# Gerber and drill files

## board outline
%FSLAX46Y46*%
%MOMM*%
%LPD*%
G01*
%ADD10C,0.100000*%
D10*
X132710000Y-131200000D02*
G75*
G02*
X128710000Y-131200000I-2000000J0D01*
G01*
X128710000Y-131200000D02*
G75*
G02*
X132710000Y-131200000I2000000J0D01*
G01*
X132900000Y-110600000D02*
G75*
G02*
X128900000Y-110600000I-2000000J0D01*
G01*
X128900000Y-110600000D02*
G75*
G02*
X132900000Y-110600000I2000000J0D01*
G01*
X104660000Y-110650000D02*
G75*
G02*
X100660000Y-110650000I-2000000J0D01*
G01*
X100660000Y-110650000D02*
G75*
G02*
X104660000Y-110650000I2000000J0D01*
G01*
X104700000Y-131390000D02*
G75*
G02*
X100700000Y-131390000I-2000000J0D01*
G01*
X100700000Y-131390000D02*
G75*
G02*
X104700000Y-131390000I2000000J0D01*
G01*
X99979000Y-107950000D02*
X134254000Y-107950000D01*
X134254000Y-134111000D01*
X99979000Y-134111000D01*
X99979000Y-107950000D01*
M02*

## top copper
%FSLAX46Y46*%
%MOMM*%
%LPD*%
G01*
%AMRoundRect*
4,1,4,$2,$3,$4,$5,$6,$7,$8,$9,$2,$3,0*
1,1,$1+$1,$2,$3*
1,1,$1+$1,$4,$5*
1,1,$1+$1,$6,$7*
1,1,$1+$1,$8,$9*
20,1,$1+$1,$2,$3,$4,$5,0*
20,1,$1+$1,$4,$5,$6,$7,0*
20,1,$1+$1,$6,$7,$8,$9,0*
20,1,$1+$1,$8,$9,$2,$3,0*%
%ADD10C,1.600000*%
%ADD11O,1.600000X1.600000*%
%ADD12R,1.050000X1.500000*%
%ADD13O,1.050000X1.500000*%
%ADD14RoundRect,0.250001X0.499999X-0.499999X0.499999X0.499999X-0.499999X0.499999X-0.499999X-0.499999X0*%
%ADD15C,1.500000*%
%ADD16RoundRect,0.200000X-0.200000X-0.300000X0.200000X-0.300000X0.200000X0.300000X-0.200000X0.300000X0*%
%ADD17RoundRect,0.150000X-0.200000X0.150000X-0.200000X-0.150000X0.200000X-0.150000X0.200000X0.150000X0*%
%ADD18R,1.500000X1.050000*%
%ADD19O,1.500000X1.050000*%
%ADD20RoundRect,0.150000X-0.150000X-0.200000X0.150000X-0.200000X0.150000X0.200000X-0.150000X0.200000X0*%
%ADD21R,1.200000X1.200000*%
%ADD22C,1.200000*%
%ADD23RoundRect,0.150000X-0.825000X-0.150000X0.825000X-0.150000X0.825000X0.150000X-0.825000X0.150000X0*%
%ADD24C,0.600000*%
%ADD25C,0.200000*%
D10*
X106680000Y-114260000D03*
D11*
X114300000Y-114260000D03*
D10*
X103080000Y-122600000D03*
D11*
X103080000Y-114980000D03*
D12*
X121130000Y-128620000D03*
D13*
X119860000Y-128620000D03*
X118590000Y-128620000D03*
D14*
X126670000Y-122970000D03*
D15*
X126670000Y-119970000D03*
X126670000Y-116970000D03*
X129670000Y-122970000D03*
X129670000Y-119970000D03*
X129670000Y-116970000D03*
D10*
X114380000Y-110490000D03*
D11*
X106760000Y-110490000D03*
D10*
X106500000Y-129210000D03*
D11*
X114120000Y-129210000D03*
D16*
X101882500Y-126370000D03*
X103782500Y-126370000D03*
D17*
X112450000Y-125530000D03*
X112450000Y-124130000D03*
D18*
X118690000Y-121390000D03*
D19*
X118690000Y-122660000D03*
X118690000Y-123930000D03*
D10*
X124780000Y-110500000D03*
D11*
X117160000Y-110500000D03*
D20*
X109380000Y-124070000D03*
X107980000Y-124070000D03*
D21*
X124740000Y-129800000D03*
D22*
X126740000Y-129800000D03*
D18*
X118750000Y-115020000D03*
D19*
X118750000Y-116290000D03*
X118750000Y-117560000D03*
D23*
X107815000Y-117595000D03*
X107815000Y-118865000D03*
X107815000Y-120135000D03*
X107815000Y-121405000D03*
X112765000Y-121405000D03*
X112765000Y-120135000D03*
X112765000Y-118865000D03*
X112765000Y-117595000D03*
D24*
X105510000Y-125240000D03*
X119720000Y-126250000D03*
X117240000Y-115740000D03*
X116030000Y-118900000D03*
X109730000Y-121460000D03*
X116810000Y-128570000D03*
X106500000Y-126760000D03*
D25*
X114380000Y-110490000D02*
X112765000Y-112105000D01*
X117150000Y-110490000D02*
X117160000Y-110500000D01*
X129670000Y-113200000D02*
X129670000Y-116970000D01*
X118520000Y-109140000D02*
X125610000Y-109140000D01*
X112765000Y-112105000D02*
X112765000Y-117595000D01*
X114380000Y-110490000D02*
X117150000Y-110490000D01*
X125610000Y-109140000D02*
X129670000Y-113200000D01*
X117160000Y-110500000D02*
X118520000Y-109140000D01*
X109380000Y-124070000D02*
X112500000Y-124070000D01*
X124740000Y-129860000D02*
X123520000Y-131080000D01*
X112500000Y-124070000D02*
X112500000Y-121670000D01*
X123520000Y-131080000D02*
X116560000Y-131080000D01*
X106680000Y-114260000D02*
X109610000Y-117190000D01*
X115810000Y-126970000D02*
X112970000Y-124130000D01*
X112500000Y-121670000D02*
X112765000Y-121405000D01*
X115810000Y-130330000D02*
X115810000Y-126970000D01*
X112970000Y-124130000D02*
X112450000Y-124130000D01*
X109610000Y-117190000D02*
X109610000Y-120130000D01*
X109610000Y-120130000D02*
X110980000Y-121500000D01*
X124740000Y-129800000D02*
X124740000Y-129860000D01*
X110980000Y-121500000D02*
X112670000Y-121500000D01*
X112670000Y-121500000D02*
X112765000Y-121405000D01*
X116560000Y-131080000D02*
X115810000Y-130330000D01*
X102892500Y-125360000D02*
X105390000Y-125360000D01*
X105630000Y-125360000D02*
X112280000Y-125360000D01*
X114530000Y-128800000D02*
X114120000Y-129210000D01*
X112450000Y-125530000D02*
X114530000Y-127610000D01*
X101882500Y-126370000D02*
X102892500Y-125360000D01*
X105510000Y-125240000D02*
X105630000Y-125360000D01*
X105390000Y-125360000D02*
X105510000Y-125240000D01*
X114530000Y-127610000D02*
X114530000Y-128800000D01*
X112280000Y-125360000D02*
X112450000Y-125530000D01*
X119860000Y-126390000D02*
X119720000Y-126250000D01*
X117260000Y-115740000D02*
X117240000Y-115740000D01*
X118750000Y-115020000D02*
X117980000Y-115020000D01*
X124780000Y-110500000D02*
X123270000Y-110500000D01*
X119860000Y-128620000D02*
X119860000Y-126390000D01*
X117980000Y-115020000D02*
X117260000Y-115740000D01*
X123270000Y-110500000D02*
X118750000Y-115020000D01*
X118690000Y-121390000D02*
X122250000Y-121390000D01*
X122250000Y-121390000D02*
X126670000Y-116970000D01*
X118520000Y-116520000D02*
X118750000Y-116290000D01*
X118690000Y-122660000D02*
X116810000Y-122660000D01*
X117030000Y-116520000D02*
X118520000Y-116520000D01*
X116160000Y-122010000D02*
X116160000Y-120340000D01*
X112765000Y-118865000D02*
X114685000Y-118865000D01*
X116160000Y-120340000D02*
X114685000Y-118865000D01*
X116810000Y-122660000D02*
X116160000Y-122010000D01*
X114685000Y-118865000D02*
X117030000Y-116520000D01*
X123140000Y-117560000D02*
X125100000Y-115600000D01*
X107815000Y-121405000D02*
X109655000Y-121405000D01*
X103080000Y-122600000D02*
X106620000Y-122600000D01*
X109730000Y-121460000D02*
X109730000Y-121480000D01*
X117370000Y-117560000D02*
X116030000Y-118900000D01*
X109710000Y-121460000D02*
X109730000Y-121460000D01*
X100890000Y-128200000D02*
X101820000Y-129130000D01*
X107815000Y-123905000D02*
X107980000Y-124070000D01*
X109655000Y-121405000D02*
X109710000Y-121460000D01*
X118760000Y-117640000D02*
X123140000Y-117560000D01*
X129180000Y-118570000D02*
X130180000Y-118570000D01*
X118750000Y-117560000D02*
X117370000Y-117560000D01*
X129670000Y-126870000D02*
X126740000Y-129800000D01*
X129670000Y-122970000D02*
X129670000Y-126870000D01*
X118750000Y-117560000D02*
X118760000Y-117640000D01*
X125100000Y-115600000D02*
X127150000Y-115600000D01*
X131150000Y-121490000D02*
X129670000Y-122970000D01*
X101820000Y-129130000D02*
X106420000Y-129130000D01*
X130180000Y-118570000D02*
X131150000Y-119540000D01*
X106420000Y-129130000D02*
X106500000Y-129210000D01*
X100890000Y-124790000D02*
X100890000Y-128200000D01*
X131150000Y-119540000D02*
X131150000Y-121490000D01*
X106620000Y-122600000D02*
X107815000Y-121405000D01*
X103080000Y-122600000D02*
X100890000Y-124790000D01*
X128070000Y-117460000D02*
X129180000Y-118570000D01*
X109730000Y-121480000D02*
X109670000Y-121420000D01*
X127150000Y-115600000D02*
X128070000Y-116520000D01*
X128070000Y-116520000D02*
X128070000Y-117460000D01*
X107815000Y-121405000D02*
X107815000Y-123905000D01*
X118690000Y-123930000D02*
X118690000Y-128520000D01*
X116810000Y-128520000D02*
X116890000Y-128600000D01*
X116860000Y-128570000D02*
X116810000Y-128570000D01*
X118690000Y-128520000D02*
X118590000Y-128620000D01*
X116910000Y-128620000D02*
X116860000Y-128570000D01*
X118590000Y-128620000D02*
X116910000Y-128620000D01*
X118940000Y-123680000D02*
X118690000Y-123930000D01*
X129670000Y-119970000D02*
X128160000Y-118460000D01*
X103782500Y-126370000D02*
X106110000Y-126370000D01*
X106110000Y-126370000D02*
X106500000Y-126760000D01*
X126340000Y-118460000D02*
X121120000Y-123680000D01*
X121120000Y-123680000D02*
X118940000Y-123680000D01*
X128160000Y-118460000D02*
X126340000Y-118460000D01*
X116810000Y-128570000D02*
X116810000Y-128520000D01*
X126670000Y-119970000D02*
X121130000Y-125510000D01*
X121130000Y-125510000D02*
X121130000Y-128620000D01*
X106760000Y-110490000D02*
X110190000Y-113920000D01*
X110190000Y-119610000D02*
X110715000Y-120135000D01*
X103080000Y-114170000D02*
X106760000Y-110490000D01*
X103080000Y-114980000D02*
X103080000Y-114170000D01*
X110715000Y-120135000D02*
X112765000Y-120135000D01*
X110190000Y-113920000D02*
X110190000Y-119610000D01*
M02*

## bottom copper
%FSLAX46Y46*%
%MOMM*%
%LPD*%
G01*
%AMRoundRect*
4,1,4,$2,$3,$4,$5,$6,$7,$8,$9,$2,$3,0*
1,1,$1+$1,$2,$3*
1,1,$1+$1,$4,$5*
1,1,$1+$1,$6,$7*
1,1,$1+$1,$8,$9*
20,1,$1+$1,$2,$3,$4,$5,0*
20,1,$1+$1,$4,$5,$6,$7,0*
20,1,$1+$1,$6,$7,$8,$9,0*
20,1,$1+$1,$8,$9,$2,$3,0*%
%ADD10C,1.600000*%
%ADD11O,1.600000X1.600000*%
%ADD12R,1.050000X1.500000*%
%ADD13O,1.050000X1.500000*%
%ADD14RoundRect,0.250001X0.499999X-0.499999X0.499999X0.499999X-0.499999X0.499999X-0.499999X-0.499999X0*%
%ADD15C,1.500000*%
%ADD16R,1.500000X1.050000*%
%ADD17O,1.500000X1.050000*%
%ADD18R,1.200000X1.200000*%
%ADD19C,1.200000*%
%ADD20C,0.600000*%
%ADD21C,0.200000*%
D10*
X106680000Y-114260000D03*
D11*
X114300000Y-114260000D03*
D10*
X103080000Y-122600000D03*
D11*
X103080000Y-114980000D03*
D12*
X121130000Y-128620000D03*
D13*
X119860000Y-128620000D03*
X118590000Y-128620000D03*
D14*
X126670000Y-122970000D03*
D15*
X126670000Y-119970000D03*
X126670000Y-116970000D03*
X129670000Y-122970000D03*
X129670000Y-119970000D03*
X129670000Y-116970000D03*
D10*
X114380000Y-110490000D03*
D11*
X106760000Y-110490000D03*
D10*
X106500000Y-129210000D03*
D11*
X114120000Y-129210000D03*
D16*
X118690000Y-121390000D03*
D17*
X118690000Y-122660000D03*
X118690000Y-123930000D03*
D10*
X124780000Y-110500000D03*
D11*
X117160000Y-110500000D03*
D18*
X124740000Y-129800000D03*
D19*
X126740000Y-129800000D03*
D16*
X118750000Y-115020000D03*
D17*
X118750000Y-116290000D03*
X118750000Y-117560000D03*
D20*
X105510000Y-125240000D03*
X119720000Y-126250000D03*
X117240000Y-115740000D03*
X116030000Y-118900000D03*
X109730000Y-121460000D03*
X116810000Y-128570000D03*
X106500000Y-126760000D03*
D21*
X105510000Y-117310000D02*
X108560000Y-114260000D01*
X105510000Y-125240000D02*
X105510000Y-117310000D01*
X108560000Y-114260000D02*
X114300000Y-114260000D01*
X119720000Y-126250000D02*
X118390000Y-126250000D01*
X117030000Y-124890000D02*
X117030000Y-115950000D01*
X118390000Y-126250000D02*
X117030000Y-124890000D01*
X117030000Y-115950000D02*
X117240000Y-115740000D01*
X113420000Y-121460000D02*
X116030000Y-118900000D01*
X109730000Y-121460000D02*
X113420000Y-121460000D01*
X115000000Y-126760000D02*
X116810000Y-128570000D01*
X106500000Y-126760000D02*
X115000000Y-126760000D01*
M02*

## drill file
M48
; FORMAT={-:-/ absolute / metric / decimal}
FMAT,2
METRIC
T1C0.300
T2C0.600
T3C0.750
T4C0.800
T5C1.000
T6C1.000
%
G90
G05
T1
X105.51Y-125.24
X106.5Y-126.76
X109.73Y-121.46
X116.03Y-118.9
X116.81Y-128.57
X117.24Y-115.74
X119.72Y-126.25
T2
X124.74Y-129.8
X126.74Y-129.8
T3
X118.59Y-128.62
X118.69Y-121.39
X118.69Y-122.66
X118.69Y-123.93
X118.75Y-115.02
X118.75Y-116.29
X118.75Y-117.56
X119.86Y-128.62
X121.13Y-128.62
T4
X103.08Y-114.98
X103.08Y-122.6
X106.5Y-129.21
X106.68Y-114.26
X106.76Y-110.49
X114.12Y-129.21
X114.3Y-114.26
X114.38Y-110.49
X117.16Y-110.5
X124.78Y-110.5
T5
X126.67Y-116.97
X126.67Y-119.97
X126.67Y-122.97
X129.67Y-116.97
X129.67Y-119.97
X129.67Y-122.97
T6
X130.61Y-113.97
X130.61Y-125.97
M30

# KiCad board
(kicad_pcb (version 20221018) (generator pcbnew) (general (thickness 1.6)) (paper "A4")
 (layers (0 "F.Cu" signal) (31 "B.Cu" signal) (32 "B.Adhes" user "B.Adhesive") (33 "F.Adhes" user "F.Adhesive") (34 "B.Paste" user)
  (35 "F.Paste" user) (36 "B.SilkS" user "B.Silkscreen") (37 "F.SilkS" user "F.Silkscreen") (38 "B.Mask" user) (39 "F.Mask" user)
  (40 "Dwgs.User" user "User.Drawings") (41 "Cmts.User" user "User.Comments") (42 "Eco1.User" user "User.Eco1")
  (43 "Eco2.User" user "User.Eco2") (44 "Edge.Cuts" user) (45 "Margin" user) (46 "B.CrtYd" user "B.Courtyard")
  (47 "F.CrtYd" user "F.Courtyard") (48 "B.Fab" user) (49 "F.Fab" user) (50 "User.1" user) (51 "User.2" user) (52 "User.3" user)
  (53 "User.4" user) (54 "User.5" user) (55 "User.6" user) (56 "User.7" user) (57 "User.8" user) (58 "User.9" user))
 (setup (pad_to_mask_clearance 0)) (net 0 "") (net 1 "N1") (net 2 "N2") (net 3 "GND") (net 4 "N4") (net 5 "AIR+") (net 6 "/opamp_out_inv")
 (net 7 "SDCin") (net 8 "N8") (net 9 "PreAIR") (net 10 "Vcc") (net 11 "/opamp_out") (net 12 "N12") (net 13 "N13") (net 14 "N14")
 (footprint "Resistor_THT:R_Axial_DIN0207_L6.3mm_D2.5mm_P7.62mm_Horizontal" (layer "F.Cu") (at 106.68 114.26)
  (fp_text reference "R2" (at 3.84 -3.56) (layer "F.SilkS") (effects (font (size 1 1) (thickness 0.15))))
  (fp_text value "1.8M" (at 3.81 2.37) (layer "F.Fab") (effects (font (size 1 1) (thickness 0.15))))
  (pad "1" thru_hole circle (at 0 0) (size 1.6 1.6) (drill 0.8) (layers "*.Cu" "*.Mask") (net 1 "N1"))
  (pad "2" thru_hole oval (at 7.62 0) (size 1.6 1.6) (drill 0.8) (layers "*.Cu" "*.Mask") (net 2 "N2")))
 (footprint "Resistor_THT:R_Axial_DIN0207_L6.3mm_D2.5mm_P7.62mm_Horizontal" (layer "F.Cu") (at 103.08 122.6 90)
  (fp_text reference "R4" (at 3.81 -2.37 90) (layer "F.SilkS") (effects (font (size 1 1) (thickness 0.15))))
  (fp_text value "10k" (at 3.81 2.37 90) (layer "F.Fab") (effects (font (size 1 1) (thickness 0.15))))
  (pad "1" thru_hole circle (at 0 0 90) (size 1.6 1.6) (drill 0.8) (layers "*.Cu" "*.Mask") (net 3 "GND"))
  (pad "2" thru_hole oval (at 7.62 0 90) (size 1.6 1.6) (drill 0.8) (layers "*.Cu" "*.Mask") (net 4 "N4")))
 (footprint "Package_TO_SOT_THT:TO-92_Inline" (layer "F.Cu") (at 121.13 128.62 180)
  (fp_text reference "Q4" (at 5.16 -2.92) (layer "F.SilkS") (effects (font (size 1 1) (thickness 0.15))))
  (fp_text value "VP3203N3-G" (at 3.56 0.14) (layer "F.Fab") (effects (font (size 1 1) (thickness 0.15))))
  (pad "1" thru_hole rect (at 0 0 180) (size 1.05 1.5) (drill 0.75) (layers "*.Cu" "*.Mask") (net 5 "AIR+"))
  (pad "2" thru_hole oval (at 1.27 0 180) (size 1.05 1.5) (drill 0.75) (layers "*.Cu" "*.Mask") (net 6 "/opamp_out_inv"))
  (pad "3" thru_hole oval (at 2.54 0 180) (size 1.05 1.5) (drill 0.75) (layers "*.Cu" "*.Mask") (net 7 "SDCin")))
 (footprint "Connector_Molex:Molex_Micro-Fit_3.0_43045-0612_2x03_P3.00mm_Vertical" (layer "F.Cu") (at 126.67 122.97 90)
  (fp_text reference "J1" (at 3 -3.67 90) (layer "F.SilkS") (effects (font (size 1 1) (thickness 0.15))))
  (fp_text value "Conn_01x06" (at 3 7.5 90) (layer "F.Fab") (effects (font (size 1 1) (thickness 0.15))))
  (pad "" np_thru_hole circle (at -3 3.94 90) (size 1 1) (drill 1) (layers "*.Cu" "*.Mask"))
  (pad "" np_thru_hole circle (at 9 3.94 90) (size 1 1) (drill 1) (layers "*.Cu" "*.Mask"))
  (pad "1" thru_hole roundrect (at 0 0 90) (size 1.5 1.5) (drill 1) (layers "*.Cu" "*.Mask") (roundrect_rratio 0.166667) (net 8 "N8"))
  (pad "2" thru_hole circle (at 3 0 90) (size 1.5 1.5) (drill 1) (layers "*.Cu" "*.Mask") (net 5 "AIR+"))
  (pad "3" thru_hole circle (at 6 0 90) (size 1.5 1.5) (drill 1) (layers "*.Cu" "*.Mask") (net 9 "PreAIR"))
  (pad "4" thru_hole circle (at 0 3 90) (size 1.5 1.5) (drill 1) (layers "*.Cu" "*.Mask") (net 3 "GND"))
  (pad "5" thru_hole circle (at 3 3 90) (size 1.5 1.5) (drill 1) (layers "*.Cu" "*.Mask") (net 7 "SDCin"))
  (pad "6" thru_hole circle (at 6 3 90) (size 1.5 1.5) (drill 1) (layers "*.Cu" "*.Mask") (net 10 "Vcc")))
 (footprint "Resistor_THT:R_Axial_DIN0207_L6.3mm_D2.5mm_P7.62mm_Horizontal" (layer "F.Cu") (at 114.38 110.49 180)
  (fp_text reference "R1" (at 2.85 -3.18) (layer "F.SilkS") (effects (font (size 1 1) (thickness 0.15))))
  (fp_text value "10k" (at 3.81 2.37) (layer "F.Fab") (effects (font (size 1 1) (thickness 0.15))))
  (pad "1" thru_hole circle (at 0 0 180) (size 1.6 1.6) (drill 0.8) (layers "*.Cu" "*.Mask") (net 10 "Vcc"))
  (pad "2" thru_hole oval (at 7.62 0 180) (size 1.6 1.6) (drill 0.8) (layers "*.Cu" "*.Mask") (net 4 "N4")))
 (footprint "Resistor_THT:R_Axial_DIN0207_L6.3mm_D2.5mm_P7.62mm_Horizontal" (layer "F.Cu") (at 106.5 129.21)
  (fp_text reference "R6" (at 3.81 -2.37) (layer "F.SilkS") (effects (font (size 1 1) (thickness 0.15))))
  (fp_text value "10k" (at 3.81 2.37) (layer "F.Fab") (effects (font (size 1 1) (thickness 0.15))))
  (pad "1" thru_hole circle (at 0 0) (size 1.6 1.6) (drill 0.8) (layers "*.Cu" "*.Mask") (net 3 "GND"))
  (pad "2" thru_hole oval (at 7.62 0) (size 1.6 1.6) (drill 0.8) (layers "*.Cu" "*.Mask") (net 2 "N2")))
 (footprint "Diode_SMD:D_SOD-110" (layer "F.Cu") (at 102.8325 126.37)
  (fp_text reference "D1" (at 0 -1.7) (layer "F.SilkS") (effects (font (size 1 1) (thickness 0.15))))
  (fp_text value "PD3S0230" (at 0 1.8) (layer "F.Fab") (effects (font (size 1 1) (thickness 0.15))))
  (pad "1" smd roundrect (at -0.95 0) (size 0.8 1) (layers "F.Cu" "F.Paste" "F.Mask") (roundrect_rratio 0.25) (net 2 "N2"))
  (pad "2" smd roundrect (at 0.95 0) (size 0.8 1) (layers "F.Cu" "F.Paste" "F.Mask") (roundrect_rratio 0.25) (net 7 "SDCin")))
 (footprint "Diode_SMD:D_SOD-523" (layer "F.Cu") (at 112.45 124.83 90)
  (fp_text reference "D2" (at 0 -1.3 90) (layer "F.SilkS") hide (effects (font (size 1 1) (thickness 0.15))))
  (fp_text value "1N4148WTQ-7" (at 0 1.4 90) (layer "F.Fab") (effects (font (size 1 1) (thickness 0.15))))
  (pad "1" smd roundrect (at -0.7 0 270) (size 0.6 0.7) (layers "F.Cu" "F.Paste" "F.Mask") (roundrect_rratio 0.25) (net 2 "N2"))
  (pad "2" smd roundrect (at 0.7 0 270) (size 0.6 0.7) (layers "F.Cu" "F.Paste" "F.Mask") (roundrect_rratio 0.25) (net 1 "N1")))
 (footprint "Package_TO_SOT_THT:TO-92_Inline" (layer "F.Cu") (at 118.69 121.39 -90)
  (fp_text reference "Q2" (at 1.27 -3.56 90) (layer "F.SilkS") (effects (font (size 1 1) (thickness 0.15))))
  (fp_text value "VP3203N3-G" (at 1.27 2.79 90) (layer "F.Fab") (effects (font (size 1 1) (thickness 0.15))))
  (pad "1" thru_hole rect (at 0 0 270) (size 1.05 1.5) (drill 0.75) (layers "*.Cu" "*.Mask") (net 9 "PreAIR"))
  (pad "2" thru_hole oval (at 1.27 0 270) (size 1.05 1.5) (drill 0.75) (layers "*.Cu" "*.Mask") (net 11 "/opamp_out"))
  (pad "3" thru_hole oval (at 2.54 0 270) (size 1.05 1.5) (drill 0.75) (layers "*.Cu" "*.Mask") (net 7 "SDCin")))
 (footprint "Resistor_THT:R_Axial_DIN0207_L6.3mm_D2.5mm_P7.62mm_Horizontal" (layer "F.Cu") (at 124.78 110.5 180)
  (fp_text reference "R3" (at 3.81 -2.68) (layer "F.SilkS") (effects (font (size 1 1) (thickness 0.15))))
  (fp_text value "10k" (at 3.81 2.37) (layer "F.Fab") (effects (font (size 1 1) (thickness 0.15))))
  (pad "1" thru_hole circle (at 0 0 180) (size 1.6 1.6) (drill 0.8) (layers "*.Cu" "*.Mask") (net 6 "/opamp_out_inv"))
  (pad "2" thru_hole oval (at 7.62 0 180) (size 1.6 1.6) (drill 0.8) (layers "*.Cu" "*.Mask") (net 10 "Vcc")))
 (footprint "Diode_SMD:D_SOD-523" (layer "F.Cu") (at 108.68 124.07 180)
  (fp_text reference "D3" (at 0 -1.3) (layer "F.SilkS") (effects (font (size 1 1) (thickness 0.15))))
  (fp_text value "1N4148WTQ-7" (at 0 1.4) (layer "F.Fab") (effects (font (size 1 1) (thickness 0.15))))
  (pad "1" smd roundrect (at -0.7 0) (size 0.6 0.7) (layers "F.Cu" "F.Paste" "F.Mask") (roundrect_rratio 0.25) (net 1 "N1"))
  (pad "2" smd roundrect (at 0.7 0) (size 0.6 0.7) (layers "F.Cu" "F.Paste" "F.Mask") (roundrect_rratio 0.25) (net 3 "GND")))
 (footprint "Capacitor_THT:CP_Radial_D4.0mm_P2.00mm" (layer "F.Cu") (at 124.74 129.8)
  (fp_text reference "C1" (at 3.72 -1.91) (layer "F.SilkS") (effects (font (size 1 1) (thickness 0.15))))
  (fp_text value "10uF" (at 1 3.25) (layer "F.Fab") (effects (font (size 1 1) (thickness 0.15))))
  (pad "1" thru_hole rect (at 0 0) (size 1.2 1.2) (drill 0.6) (layers "*.Cu" "*.Mask") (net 1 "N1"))
  (pad "2" thru_hole circle (at 2 0) (size 1.2 1.2) (drill 0.6) (layers "*.Cu" "*.Mask") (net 3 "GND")))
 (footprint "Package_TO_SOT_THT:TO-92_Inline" (layer "F.Cu") (at 118.75 115.02 -90)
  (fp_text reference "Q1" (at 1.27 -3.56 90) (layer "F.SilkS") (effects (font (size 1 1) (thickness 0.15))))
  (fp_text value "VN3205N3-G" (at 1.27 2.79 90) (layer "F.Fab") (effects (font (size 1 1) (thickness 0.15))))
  (pad "1" thru_hole rect (at 0 0 270) (size 1.05 1.5) (drill 0.75) (layers "*.Cu" "*.Mask") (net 6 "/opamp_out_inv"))
  (pad "2" thru_hole oval (at 1.27 0 270) (size 1.05 1.5) (drill 0.75) (layers "*.Cu" "*.Mask") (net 11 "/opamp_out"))
  (pad "3" thru_hole oval (at 2.54 0 270) (size 1.05 1.5) (drill 0.75) (layers "*.Cu" "*.Mask") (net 3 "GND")))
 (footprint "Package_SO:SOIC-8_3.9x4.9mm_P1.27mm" (layer "F.Cu") (at 110.29 119.5)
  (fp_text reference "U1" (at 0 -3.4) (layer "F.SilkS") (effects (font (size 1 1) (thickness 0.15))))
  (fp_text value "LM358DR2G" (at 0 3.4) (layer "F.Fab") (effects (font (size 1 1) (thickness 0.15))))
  (pad "1" smd roundrect (at -2.475 -1.905) (size 1.95 0.6) (layers "F.Cu" "F.Paste" "F.Mask") (roundrect_rratio 0.25) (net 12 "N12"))
  (pad "2" smd roundrect (at -2.475 -0.635) (size 1.95 0.6) (layers "F.Cu" "F.Paste" "F.Mask") (roundrect_rratio 0.25) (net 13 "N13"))
  (pad "3" smd roundrect (at -2.475 0.635) (size 1.95 0.6) (layers "F.Cu" "F.Paste" "F.Mask") (roundrect_rratio 0.25) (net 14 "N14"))
  (pad "4" smd roundrect (at -2.475 1.905) (size 1.95 0.6) (layers "F.Cu" "F.Paste" "F.Mask") (roundrect_rratio 0.25) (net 3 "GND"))
  (pad "5" smd roundrect (at 2.475 1.905) (size 1.95 0.6) (layers "F.Cu" "F.Paste" "F.Mask") (roundrect_rratio 0.25) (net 1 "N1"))
  (pad "6" smd roundrect (at 2.475 0.635) (size 1.95 0.6) (layers "F.Cu" "F.Paste" "F.Mask") (roundrect_rratio 0.25) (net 4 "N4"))
  (pad "7" smd roundrect (at 2.475 -0.635) (size 1.95 0.6) (layers "F.Cu" "F.Paste" "F.Mask") (roundrect_rratio 0.25) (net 11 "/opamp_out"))
  (pad "8" smd roundrect (at 2.475 -1.905) (size 1.95 0.6) (layers "F.Cu" "F.Paste" "F.Mask") (roundrect_rratio 0.25) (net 10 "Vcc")))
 (gr_circle (center 130.71 131.2) (end 132.71 131.2) (stroke (width 0.1) (type default)) (fill none) (layer "Edge.Cuts"))
 (gr_circle (center 130.9 110.6) (end 132.9 110.6) (stroke (width 0.1) (type default)) (fill none) (layer "Edge.Cuts"))
 (gr_circle (center 102.66 110.65) (end 104.66 110.65) (stroke (width 0.1) (type default)) (fill none) (layer "Edge.Cuts"))
 (gr_circle (center 102.7 131.39) (end 104.7 131.39) (stroke (width 0.1) (type default)) (fill none) (layer "Edge.Cuts"))
 (gr_rect (start 99.979 107.95) (end 134.254 134.111) (stroke (width 0.1) (type solid)) (fill none) (layer "Edge.Cuts"))
 (segment (start 114.38 110.49) (end 112.765 112.105) (width 0.2) (layer "F.Cu") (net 10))
 (segment (start 117.15 110.49) (end 117.16 110.5) (width 0.2) (layer "F.Cu") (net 10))
 (segment (start 129.67 113.2) (end 129.67 116.97) (width 0.2) (layer "F.Cu") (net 10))
 (segment (start 118.52 109.14) (end 125.61 109.14) (width 0.2) (layer "F.Cu") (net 10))
 (segment (start 112.765 112.105) (end 112.765 117.595) (width 0.2) (layer "F.Cu") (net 10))
 (segment (start 114.38 110.49) (end 117.15 110.49) (width 0.2) (layer "F.Cu") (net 10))
 (segment (start 125.61 109.14) (end 129.67 113.2) (width 0.2) (layer "F.Cu") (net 10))
 (segment (start 117.16 110.5) (end 118.52 109.14) (width 0.2) (layer "F.Cu") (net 10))
 (segment (start 109.38 124.07) (end 112.5 124.07) (width 0.2) (layer "F.Cu") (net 1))
 (segment (start 124.74 129.86) (end 123.52 131.08) (width 0.2) (layer "F.Cu") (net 1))
 (segment (start 112.5 124.07) (end 112.5 121.67) (width 0.2) (layer "F.Cu") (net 1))
 (segment (start 123.52 131.08) (end 116.56 131.08) (width 0.2) (layer "F.Cu") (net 1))
 (segment (start 106.68 114.26) (end 109.61 117.19) (width 0.2) (layer "F.Cu") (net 1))
 (segment (start 115.81 126.97) (end 112.97 124.13) (width 0.2) (layer "F.Cu") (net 1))
 (segment (start 112.5 121.67) (end 112.765 121.405) (width 0.2) (layer "F.Cu") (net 1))
 (segment (start 115.81 130.33) (end 115.81 126.97) (width 0.2) (layer "F.Cu") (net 1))
 (segment (start 112.97 124.13) (end 112.45 124.13) (width 0.2) (layer "F.Cu") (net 1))
 (segment (start 109.61 117.19) (end 109.61 120.13) (width 0.2) (layer "F.Cu") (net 1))
 (segment (start 109.61 120.13) (end 110.98 121.5) (width 0.2) (layer "F.Cu") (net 1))
 (segment (start 124.74 129.8) (end 124.74 129.86) (width 0.2) (layer "F.Cu") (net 1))
 (segment (start 110.98 121.5) (end 112.67 121.5) (width 0.2) (layer "F.Cu") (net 1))
 (segment (start 112.67 121.5) (end 112.765 121.405) (width 0.2) (layer "F.Cu") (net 1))
 (segment (start 116.56 131.08) (end 115.81 130.33) (width 0.2) (layer "F.Cu") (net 1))
 (segment (start 102.8925 125.36) (end 105.39 125.36) (width 0.2) (layer "F.Cu") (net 2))
 (segment (start 105.63 125.36) (end 112.28 125.36) (width 0.2) (layer "F.Cu") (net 2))
 (segment (start 114.53 128.8) (end 114.12 129.21) (width 0.2) (layer "F.Cu") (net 2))
 (segment (start 112.45 125.53) (end 114.53 127.61) (width 0.2) (layer "F.Cu") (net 2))
 (segment (start 101.8825 126.37) (end 102.8925 125.36) (width 0.2) (layer "F.Cu") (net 2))
 (segment (start 105.51 125.24) (end 105.63 125.36) (width 0.2) (layer "F.Cu") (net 2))
 (segment (start 105.39 125.36) (end 105.51 125.24) (width 0.2) (layer "F.Cu") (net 2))
 (segment (start 114.53 127.61) (end 114.53 128.8) (width 0.2) (layer "F.Cu") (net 2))
 (segment (start 112.28 125.36) (end 112.45 125.53) (width 0.2) (layer "F.Cu") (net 2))
 (via (at 105.51 125.24) (size 0.6) (drill 0.3) (layers "F.Cu" "B.Cu") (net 2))
 (segment (start 105.51 117.31) (end 108.56 114.26) (width 0.2) (layer "B.Cu") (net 2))
 (segment (start 105.51 125.24) (end 105.51 117.31) (width 0.2) (layer "B.Cu") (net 2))
 (segment (start 108.56 114.26) (end 114.3 114.26) (width 0.2) (layer "B.Cu") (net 2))
 (segment (start 119.86 126.39) (end 119.72 126.25) (width 0.2) (layer "F.Cu") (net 6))
 (segment (start 117.26 115.74) (end 117.24 115.74) (width 0.2) (layer "F.Cu") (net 6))
 (segment (start 118.75 115.02) (end 117.98 115.02) (width 0.2) (layer "F.Cu") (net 6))
 (segment (start 124.78 110.5) (end 123.27 110.5) (width 0.2) (layer "F.Cu") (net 6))
 (segment (start 119.86 128.62) (end 119.86 126.39) (width 0.2) (layer "F.Cu") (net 6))
 (segment (start 117.98 115.02) (end 117.26 115.74) (width 0.2) (layer "F.Cu") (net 6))
 (segment (start 123.27 110.5) (end 118.75 115.02) (width 0.2) (layer "F.Cu") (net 6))
 (via (at 119.72 126.25) (size 0.6) (drill 0.3) (layers "F.Cu" "B.Cu") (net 6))
 (via (at 117.24 115.74) (size 0.6) (drill 0.3) (layers "F.Cu" "B.Cu") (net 6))
 (segment (start 119.72 126.25) (end 118.39 126.25) (width 0.2) (layer "B.Cu") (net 6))
 (segment (start 117.03 124.89) (end 117.03 115.95) (width 0.2) (layer "B.Cu") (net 6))
 (segment (start 118.39 126.25) (end 117.03 124.89) (width 0.2) (layer "B.Cu") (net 6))
 (segment (start 117.03 115.95) (end 117.24 115.74) (width 0.2) (layer "B.Cu") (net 6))
 (segment (start 118.69 121.39) (end 122.25 121.39) (width 0.2) (layer "F.Cu") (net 9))
 (segment (start 122.25 121.39) (end 126.67 116.97) (width 0.2) (layer "F.Cu") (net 9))
 (segment (start 118.52 116.52) (end 118.75 116.29) (width 0.2) (layer "F.Cu") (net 11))
 (segment (start 118.69 122.66) (end 116.81 122.66) (width 0.2) (layer "F.Cu") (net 11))
 (segment (start 117.03 116.52) (end 118.52 116.52) (width 0.2) (layer "F.Cu") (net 11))
 (segment (start 116.16 122.01) (end 116.16 120.34) (width 0.2) (layer "F.Cu") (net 11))
 (segment (start 112.765 118.865) (end 114.685 118.865) (width 0.2) (layer "F.Cu") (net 11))
 (segment (start 116.16 120.34) (end 114.685 118.865) (width 0.2) (layer "F.Cu") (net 11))
 (segment (start 116.81 122.66) (end 116.16 122.01) (width 0.2) (layer "F.Cu") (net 11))
 (segment (start 114.685 118.865) (end 117.03 116.52) (width 0.2) (layer "F.Cu") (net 11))
 (segment (start 123.14 117.56) (end 125.1 115.6) (width 0.2) (layer "F.Cu") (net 3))
 (segment (start 107.815 121.405) (end 109.655 121.405) (width 0.2) (layer "F.Cu") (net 3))
 (segment (start 103.08 122.6) (end 106.62 122.6) (width 0.2) (layer "F.Cu") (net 3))
 (segment (start 109.73 121.46) (end 109.73 121.48) (width 0.2) (layer "F.Cu") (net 3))
 (segment (start 117.37 117.56) (end 116.03 118.9) (width 0.2) (layer "F.Cu") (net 3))
 (segment (start 109.71 121.46) (end 109.73 121.46) (width 0.2) (layer "F.Cu") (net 3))
 (segment (start 100.89 128.2) (end 101.82 129.13) (width 0.2) (layer "F.Cu") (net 3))
 (segment (start 107.815 123.905) (end 107.98 124.07) (width 0.2) (layer "F.Cu") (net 3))
 (segment (start 109.655 121.405) (end 109.71 121.46) (width 0.2) (layer "F.Cu") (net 3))
 (segment (start 118.76 117.64) (end 123.14 117.56) (width 0.2) (layer "F.Cu") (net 3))
 (segment (start 129.18 118.57) (end 130.18 118.57) (width 0.2) (layer "F.Cu") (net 3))
 (segment (start 118.75 117.56) (end 117.37 117.56) (width 0.2) (layer "F.Cu") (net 3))
 (segment (start 129.67 126.87) (end 126.74 129.8) (width 0.2) (layer "F.Cu") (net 3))
 (segment (start 129.67 122.97) (end 129.67 126.87) (width 0.2) (layer "F.Cu") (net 3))
 (segment (start 118.75 117.56) (end 118.76 117.64) (width 0.2) (layer "F.Cu") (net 3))
 (segment (start 125.1 115.6) (end 127.15 115.6) (width 0.2) (layer "F.Cu") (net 3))
 (segment (start 131.15 121.49) (end 129.67 122.97) (width 0.2) (layer "F.Cu") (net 3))
 (segment (start 101.82 129.13) (end 106.42 129.13) (width 0.2) (layer "F.Cu") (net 3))
 (segment (start 130.18 118.57) (end 131.15 119.54) (width 0.2) (layer "F.Cu") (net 3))
 (segment (start 106.42 129.13) (end 106.5 129.21) (width 0.2) (layer "F.Cu") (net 3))
 (segment (start 100.89 124.79) (end 100.89 128.2) (width 0.2) (layer "F.Cu") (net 3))
 (segment (start 131.15 119.54) (end 131.15 121.49) (width 0.2) (layer "F.Cu") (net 3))
 (segment (start 106.62 122.6) (end 107.815 121.405) (width 0.2) (layer "F.Cu") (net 3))
 (segment (start 103.08 122.6) (end 100.89 124.79) (width 0.2) (layer "F.Cu") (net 3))
 (segment (start 128.07 117.46) (end 129.18 118.57) (width 0.2) (layer "F.Cu") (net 3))
 (segment (start 109.73 121.48) (end 109.67 121.42) (width 0.2) (layer "F.Cu") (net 3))
 (segment (start 127.15 115.6) (end 128.07 116.52) (width 0.2) (layer "F.Cu") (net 3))
 (segment (start 128.07 116.52) (end 128.07 117.46) (width 0.2) (layer "F.Cu") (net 3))
 (segment (start 107.815 121.405) (end 107.815 123.905) (width 0.2) (layer "F.Cu") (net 3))
 (via (at 116.03 118.9) (size 0.6) (drill 0.3) (layers "F.Cu" "B.Cu") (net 3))
 (via (at 109.73 121.46) (size 0.6) (drill 0.3) (layers "F.Cu" "B.Cu") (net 3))
 (segment (start 113.42 121.46) (end 116.03 118.9) (width 0.2) (layer "B.Cu") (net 3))
 (segment (start 109.73 121.46) (end 113.42 121.46) (width 0.2) (layer "B.Cu") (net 3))
 (segment (start 118.69 123.93) (end 118.69 128.52) (width 0.2) (layer "F.Cu") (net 7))
 (segment (start 116.81 128.52) (end 116.89 128.6) (width 0.2) (layer "F.Cu") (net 7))
 (segment (start 116.86 128.57) (end 116.81 128.57) (width 0.2) (layer "F.Cu") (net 7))
 (segment (start 118.69 128.52) (end 118.59 128.62) (width 0.2) (layer "F.Cu") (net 7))
 (segment (start 116.91 128.62) (end 116.86 128.57) (width 0.2) (layer "F.Cu") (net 7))
 (segment (start 118.59 128.62) (end 116.91 128.62) (width 0.2) (layer "F.Cu") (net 7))
 (segment (start 118.94 123.68) (end 118.69 123.93) (width 0.2) (layer "F.Cu") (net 7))
 (segment (start 129.67 119.97) (end 128.16 118.46) (width 0.2) (layer "F.Cu") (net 7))
 (segment (start 103.7825 126.37) (end 106.11 126.37) (width 0.2) (layer "F.Cu") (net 7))
 (segment (start 106.11 126.37) (end 106.5 126.76) (width 0.2) (layer "F.Cu") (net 7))
 (segment (start 126.34 118.46) (end 121.12 123.68) (width 0.2) (layer "F.Cu") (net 7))
 (segment (start 121.12 123.68) (end 118.94 123.68) (width 0.2) (layer "F.Cu") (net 7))
 (segment (start 128.16 118.46) (end 126.34 118.46) (width 0.2) (layer "F.Cu") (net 7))
 (segment (start 116.81 128.57) (end 116.81 128.52) (width 0.2) (layer "F.Cu") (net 7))
 (via (at 116.81 128.57) (size 0.6) (drill 0.3) (layers "F.Cu" "B.Cu") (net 7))
 (via (at 106.5 126.76) (size 0.6) (drill 0.3) (layers "F.Cu" "B.Cu") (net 7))
 (segment (start 115 126.76) (end 116.81 128.57) (width 0.2) (layer "B.Cu") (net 7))
 (segment (start 106.5 126.76) (end 115 126.76) (width 0.2) (layer "B.Cu") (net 7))
 (segment (start 126.67 119.97) (end 121.13 125.51) (width 0.2) (layer "F.Cu") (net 5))
 (segment (start 121.13 125.51) (end 121.13 128.62) (width 0.2) (layer "F.Cu") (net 5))
 (segment (start 106.76 110.49) (end 110.19 113.92) (width 0.2) (layer "F.Cu") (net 4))
 (segment (start 110.19 119.61) (end 110.715 120.135) (width 0.2) (layer "F.Cu") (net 4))
 (segment (start 103.08 114.17) (end 106.76 110.49) (width 0.2) (layer "F.Cu") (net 4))
 (segment (start 103.08 114.98) (end 103.08 114.17) (width 0.2) (layer "F.Cu") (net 4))
 (segment (start 110.715 120.135) (end 112.765 120.135) (width 0.2) (layer "F.Cu") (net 4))
 (segment (start 110.19 113.92) (end 110.19 119.61) (width 0.2) (layer "F.Cu") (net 4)))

